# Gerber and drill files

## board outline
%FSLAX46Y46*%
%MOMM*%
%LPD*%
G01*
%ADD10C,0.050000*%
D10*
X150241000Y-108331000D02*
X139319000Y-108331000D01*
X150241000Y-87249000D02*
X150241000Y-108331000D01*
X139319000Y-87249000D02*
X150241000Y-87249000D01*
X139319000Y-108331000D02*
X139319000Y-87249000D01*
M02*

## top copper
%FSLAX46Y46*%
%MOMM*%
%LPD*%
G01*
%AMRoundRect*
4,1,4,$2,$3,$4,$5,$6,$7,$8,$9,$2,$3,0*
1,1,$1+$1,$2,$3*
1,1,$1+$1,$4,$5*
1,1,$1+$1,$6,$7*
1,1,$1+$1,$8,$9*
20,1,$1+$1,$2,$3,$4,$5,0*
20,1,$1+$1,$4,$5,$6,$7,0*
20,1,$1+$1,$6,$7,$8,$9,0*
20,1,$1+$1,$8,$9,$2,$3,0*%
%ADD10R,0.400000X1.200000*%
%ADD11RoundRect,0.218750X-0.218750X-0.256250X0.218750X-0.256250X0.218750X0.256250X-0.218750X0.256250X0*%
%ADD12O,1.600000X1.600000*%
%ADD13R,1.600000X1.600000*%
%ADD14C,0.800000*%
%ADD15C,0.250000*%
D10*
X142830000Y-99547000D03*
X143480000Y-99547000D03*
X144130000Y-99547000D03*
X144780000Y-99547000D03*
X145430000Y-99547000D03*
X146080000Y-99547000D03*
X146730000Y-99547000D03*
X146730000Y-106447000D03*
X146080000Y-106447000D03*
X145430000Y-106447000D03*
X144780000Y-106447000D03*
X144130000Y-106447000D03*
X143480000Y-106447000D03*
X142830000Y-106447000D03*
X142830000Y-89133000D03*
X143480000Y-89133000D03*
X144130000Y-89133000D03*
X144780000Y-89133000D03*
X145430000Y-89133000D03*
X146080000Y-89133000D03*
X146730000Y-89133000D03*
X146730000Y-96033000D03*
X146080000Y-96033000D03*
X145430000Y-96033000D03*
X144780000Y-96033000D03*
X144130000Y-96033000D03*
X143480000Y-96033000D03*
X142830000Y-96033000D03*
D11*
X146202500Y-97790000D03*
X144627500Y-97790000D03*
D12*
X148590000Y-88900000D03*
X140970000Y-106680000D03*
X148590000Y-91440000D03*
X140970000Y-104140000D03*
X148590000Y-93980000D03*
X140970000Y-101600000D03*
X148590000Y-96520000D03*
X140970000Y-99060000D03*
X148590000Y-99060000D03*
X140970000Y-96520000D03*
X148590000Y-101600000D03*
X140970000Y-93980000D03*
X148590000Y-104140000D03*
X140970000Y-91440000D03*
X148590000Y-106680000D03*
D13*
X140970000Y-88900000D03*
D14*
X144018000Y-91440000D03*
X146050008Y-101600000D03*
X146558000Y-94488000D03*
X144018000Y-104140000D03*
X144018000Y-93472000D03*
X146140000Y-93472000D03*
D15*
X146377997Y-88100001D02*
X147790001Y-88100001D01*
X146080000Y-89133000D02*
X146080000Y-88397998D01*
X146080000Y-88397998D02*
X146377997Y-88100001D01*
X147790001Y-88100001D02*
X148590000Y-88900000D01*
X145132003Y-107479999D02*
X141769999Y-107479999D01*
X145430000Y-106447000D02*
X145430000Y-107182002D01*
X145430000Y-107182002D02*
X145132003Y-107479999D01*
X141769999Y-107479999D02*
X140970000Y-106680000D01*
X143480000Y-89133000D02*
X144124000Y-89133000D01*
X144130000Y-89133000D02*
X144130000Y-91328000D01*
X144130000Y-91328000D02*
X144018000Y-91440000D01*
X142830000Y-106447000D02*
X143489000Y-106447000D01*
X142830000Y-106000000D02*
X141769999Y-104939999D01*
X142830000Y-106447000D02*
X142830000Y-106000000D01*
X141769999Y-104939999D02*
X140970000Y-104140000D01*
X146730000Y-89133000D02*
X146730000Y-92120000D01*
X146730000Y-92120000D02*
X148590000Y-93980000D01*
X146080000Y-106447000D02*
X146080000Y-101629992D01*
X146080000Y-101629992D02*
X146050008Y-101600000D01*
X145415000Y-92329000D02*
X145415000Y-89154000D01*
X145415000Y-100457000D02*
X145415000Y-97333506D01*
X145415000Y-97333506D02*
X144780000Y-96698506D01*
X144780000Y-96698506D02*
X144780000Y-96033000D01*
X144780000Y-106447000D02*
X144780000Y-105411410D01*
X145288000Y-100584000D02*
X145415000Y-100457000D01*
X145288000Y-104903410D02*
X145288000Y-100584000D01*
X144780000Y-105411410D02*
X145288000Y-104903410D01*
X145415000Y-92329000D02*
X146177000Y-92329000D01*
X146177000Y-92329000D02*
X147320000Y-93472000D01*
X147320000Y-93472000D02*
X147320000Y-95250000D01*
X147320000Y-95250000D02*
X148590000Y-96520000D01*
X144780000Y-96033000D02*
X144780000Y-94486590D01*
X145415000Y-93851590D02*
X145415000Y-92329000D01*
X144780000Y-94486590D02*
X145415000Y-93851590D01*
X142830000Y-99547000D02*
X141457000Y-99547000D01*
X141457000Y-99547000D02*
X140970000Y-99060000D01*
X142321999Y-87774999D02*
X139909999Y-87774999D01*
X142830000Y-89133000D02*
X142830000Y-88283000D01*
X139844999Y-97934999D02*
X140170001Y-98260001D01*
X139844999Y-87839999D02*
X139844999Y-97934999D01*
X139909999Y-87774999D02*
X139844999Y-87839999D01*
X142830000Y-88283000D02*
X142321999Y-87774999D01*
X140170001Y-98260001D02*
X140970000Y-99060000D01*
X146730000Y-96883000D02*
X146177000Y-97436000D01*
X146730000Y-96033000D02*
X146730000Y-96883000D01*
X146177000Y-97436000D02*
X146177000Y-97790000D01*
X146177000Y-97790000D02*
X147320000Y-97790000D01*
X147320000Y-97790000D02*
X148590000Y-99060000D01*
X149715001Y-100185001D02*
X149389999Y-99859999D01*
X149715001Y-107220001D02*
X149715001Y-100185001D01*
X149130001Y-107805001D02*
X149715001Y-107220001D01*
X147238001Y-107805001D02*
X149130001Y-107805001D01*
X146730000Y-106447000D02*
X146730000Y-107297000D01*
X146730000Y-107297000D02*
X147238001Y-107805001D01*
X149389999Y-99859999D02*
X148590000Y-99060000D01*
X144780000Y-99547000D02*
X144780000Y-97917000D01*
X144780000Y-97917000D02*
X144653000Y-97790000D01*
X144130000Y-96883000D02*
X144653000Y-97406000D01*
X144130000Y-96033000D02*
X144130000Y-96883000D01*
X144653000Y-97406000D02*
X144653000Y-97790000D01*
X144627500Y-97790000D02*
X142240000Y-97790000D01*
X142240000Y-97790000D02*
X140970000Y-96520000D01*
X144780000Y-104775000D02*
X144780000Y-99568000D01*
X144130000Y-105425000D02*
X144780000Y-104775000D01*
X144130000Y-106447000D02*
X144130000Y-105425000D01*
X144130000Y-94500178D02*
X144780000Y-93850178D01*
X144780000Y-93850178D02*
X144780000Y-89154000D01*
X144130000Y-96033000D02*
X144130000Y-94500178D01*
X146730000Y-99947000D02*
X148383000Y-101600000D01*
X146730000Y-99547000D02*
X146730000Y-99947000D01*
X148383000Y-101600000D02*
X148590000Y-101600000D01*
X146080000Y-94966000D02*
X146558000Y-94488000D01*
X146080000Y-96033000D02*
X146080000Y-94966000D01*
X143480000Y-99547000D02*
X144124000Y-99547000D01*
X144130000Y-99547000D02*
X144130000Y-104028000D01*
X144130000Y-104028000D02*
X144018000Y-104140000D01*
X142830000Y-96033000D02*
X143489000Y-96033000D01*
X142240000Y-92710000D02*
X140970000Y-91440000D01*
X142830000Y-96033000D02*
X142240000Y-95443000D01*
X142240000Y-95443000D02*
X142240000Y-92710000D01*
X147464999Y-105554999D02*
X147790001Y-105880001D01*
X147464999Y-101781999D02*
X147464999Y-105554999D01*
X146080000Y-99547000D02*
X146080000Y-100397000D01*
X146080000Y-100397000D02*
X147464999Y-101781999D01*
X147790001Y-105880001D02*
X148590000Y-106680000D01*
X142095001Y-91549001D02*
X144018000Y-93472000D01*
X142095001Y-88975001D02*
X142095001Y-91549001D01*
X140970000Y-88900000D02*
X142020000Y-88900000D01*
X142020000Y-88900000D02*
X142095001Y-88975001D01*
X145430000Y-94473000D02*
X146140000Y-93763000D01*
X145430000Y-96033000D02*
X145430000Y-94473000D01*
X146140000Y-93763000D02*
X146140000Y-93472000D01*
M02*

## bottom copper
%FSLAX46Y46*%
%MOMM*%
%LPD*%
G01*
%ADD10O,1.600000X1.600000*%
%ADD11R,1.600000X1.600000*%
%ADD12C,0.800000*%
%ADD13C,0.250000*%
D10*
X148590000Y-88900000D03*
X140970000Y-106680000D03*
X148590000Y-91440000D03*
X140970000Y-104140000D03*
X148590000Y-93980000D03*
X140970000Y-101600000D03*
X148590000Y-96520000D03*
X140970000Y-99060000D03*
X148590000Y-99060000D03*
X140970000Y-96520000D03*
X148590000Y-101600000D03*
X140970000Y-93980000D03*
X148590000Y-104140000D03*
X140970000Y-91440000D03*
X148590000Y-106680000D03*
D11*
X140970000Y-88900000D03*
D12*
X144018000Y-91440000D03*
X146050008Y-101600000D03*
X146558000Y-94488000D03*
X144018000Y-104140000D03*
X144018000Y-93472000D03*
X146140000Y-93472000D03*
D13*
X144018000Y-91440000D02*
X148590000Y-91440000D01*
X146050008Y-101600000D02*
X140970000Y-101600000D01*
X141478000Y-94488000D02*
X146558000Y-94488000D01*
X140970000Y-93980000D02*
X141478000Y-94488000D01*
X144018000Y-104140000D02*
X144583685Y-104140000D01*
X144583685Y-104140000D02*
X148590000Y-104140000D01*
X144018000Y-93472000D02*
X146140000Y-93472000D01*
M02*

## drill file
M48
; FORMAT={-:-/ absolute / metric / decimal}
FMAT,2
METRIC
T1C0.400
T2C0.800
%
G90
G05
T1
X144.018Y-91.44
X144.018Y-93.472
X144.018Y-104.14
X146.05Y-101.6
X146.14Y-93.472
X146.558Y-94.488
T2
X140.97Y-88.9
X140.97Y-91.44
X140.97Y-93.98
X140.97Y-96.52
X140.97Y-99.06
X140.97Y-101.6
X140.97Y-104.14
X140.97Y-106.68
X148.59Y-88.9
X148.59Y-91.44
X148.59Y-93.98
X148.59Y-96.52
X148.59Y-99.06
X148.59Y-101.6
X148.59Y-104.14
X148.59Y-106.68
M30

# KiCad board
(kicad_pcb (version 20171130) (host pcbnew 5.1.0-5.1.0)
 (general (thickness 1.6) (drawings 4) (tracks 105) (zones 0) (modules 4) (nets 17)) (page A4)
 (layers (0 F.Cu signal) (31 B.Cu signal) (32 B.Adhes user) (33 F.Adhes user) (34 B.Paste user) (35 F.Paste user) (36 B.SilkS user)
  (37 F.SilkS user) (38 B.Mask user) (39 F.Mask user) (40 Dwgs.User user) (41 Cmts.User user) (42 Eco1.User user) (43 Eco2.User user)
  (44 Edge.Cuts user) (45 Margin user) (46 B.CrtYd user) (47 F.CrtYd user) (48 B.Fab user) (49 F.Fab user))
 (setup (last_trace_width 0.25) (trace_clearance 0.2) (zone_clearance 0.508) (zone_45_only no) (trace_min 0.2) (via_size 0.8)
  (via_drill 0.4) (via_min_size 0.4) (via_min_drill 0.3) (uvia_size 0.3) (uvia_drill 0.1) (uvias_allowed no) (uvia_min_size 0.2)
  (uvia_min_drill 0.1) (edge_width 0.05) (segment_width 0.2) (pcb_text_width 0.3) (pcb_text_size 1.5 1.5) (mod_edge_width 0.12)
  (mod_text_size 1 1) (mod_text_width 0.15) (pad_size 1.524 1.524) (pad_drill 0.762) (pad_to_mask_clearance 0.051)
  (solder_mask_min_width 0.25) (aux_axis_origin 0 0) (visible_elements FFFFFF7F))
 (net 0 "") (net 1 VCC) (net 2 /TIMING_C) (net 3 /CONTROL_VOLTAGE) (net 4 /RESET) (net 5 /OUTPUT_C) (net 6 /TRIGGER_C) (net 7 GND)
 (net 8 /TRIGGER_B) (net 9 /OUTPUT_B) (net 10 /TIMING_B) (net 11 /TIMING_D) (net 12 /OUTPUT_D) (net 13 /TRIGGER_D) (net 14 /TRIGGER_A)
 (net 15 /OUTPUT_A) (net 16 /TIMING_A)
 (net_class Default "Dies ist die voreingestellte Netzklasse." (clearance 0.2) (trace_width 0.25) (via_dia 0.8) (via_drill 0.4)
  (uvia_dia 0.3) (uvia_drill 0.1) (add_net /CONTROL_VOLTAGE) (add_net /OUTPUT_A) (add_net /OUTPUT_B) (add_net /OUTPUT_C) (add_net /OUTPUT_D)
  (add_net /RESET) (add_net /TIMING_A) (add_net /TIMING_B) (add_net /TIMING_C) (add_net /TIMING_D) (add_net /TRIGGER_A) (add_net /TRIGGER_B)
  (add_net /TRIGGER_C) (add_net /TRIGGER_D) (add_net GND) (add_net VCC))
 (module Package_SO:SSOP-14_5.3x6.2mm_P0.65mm (layer F.Cu) (at 144.78 102.997 90)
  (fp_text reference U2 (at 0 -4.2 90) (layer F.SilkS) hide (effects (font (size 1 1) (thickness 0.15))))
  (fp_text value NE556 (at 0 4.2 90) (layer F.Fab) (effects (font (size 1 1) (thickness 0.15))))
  (pad 14 smd rect (at 3.45 -1.95 90) (size 1.2 0.4) (layers F.Cu F.Paste F.Mask) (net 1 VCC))
  (pad 13 smd rect (at 3.45 -1.3 90) (size 1.2 0.4) (layers F.Cu F.Paste F.Mask) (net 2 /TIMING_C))
  (pad 12 smd rect (at 3.45 -0.65 90) (size 1.2 0.4) (layers F.Cu F.Paste F.Mask) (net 2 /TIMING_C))
  (pad 11 smd rect (at 3.45 0 90) (size 1.2 0.4) (layers F.Cu F.Paste F.Mask) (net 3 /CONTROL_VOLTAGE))
  (pad 10 smd rect (at 3.45 0.65 90) (size 1.2 0.4) (layers F.Cu F.Paste F.Mask) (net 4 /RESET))
  (pad 9 smd rect (at 3.45 1.3 90) (size 1.2 0.4) (layers F.Cu F.Paste F.Mask) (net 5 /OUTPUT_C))
  (pad 8 smd rect (at 3.45 1.95 90) (size 1.2 0.4) (layers F.Cu F.Paste F.Mask) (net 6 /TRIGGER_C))
  (pad 7 smd rect (at -3.45 1.95 90) (size 1.2 0.4) (layers F.Cu F.Paste F.Mask) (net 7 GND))
  (pad 6 smd rect (at -3.45 1.3 90) (size 1.2 0.4) (layers F.Cu F.Paste F.Mask) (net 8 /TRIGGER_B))
  (pad 5 smd rect (at -3.45 0.65 90) (size 1.2 0.4) (layers F.Cu F.Paste F.Mask) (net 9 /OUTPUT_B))
  (pad 4 smd rect (at -3.45 0 90) (size 1.2 0.4) (layers F.Cu F.Paste F.Mask) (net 4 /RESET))
  (pad 3 smd rect (at -3.45 -0.65 90) (size 1.2 0.4) (layers F.Cu F.Paste F.Mask) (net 3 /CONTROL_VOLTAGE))
  (pad 2 smd rect (at -3.45 -1.3 90) (size 1.2 0.4) (layers F.Cu F.Paste F.Mask) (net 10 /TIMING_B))
  (pad 1 smd rect (at -3.45 -1.95 90) (size 1.2 0.4) (layers F.Cu F.Paste F.Mask) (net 10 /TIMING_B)))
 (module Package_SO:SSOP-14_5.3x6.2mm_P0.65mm (layer F.Cu) (at 144.78 92.583 90)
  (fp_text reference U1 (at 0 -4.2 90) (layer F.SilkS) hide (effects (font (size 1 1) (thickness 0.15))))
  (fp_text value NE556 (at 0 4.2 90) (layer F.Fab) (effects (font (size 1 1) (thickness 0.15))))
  (pad 14 smd rect (at 3.45 -1.95 90) (size 1.2 0.4) (layers F.Cu F.Paste F.Mask) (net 1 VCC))
  (pad 13 smd rect (at 3.45 -1.3 90) (size 1.2 0.4) (layers F.Cu F.Paste F.Mask) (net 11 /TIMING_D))
  (pad 12 smd rect (at 3.45 -0.65 90) (size 1.2 0.4) (layers F.Cu F.Paste F.Mask) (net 11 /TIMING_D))
  (pad 11 smd rect (at 3.45 0 90) (size 1.2 0.4) (layers F.Cu F.Paste F.Mask) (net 3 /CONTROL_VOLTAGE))
  (pad 10 smd rect (at 3.45 0.65 90) (size 1.2 0.4) (layers F.Cu F.Paste F.Mask) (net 4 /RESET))
  (pad 9 smd rect (at 3.45 1.3 90) (size 1.2 0.4) (layers F.Cu F.Paste F.Mask) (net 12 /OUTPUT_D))
  (pad 8 smd rect (at 3.45 1.95 90) (size 1.2 0.4) (layers F.Cu F.Paste F.Mask) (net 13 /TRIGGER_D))
  (pad 7 smd rect (at -3.45 1.95 90) (size 1.2 0.4) (layers F.Cu F.Paste F.Mask) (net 7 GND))
  (pad 6 smd rect (at -3.45 1.3 90) (size 1.2 0.4) (layers F.Cu F.Paste F.Mask) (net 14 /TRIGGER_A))
  (pad 5 smd rect (at -3.45 0.65 90) (size 1.2 0.4) (layers F.Cu F.Paste F.Mask) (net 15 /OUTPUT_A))
  (pad 4 smd rect (at -3.45 0 90) (size 1.2 0.4) (layers F.Cu F.Paste F.Mask) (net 4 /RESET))
  (pad 3 smd rect (at -3.45 -0.65 90) (size 1.2 0.4) (layers F.Cu F.Paste F.Mask) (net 3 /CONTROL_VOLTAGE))
  (pad 2 smd rect (at -3.45 -1.3 90) (size 1.2 0.4) (layers F.Cu F.Paste F.Mask) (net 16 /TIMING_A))
  (pad 1 smd rect (at -3.45 -1.95 90) (size 1.2 0.4) (layers F.Cu F.Paste F.Mask) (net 16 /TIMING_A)))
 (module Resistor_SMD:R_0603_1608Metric (layer F.Cu) (at 145.415 97.79)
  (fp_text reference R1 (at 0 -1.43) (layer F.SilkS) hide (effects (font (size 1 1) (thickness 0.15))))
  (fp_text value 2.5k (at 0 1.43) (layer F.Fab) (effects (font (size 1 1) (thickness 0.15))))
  (pad 2 smd roundrect (at 0.7875 0) (size 0.875 0.95) (layers F.Cu F.Paste F.Mask) (roundrect_rratio 0.25) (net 7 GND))
  (pad 1 smd roundrect (at -0.7875 0) (size 0.875 0.95) (layers F.Cu F.Paste F.Mask) (roundrect_rratio 0.25) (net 3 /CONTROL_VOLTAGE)))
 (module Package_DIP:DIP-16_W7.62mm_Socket (layer F.Cu) (at 140.97 88.9)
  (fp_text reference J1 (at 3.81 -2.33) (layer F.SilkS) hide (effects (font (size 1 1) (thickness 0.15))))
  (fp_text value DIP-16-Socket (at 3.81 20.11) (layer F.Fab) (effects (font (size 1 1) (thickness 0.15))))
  (pad 16 thru_hole oval (at 7.62 0) (size 1.6 1.6) (drill 0.8) (layers *.Cu *.Mask) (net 12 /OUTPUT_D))
  (pad 8 thru_hole oval (at 0 17.78) (size 1.6 1.6) (drill 0.8) (layers *.Cu *.Mask) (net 9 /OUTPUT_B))
  (pad 15 thru_hole oval (at 7.62 2.54) (size 1.6 1.6) (drill 0.8) (layers *.Cu *.Mask) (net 11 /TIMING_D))
  (pad 7 thru_hole oval (at 0 15.24) (size 1.6 1.6) (drill 0.8) (layers *.Cu *.Mask) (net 10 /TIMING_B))
  (pad 14 thru_hole oval (at 7.62 5.08) (size 1.6 1.6) (drill 0.8) (layers *.Cu *.Mask) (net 13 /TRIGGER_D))
  (pad 6 thru_hole oval (at 0 12.7) (size 1.6 1.6) (drill 0.8) (layers *.Cu *.Mask) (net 8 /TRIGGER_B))
  (pad 13 thru_hole oval (at 7.62 7.62) (size 1.6 1.6) (drill 0.8) (layers *.Cu *.Mask) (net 4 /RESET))
  (pad 5 thru_hole oval (at 0 10.16) (size 1.6 1.6) (drill 0.8) (layers *.Cu *.Mask) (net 1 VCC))
  (pad 12 thru_hole oval (at 7.62 10.16) (size 1.6 1.6) (drill 0.8) (layers *.Cu *.Mask) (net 7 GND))
  (pad 4 thru_hole oval (at 0 7.62) (size 1.6 1.6) (drill 0.8) (layers *.Cu *.Mask) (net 3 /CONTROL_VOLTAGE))
  (pad 11 thru_hole oval (at 7.62 12.7) (size 1.6 1.6) (drill 0.8) (layers *.Cu *.Mask) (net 6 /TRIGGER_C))
  (pad 3 thru_hole oval (at 0 5.08) (size 1.6 1.6) (drill 0.8) (layers *.Cu *.Mask) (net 14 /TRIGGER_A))
  (pad 10 thru_hole oval (at 7.62 15.24) (size 1.6 1.6) (drill 0.8) (layers *.Cu *.Mask) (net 2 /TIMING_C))
  (pad 2 thru_hole oval (at 0 2.54) (size 1.6 1.6) (drill 0.8) (layers *.Cu *.Mask) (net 16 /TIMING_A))
  (pad 9 thru_hole oval (at 7.62 17.78) (size 1.6 1.6) (drill 0.8) (layers *.Cu *.Mask) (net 5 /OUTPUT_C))
  (pad 1 thru_hole rect (at 0 0) (size 1.6 1.6) (drill 0.8) (layers *.Cu *.Mask) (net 15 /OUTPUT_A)))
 (gr_line (start 150.241 108.331) (end 139.319 108.331) (layer Edge.Cuts) (width 0.05))
 (gr_line (start 150.241 87.249) (end 150.241 108.331) (layer Edge.Cuts) (width 0.05))
 (gr_line (start 139.319 87.249) (end 150.241 87.249) (layer Edge.Cuts) (width 0.05))
 (gr_line (start 139.319 108.331) (end 139.319 87.249) (layer Edge.Cuts) (width 0.05))
 (segment (start 146.377997 88.100001) (end 147.790001 88.100001) (width 0.25) (layer F.Cu) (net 12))
 (segment (start 146.08 89.133) (end 146.08 88.397998) (width 0.25) (layer F.Cu) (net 12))
 (segment (start 146.08 88.397998) (end 146.377997 88.100001) (width 0.25) (layer F.Cu) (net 12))
 (segment (start 147.790001 88.100001) (end 148.59 88.9) (width 0.25) (layer F.Cu) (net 12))
 (segment (start 145.132003 107.479999) (end 141.769999 107.479999) (width 0.25) (layer F.Cu) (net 9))
 (segment (start 145.43 106.447) (end 145.43 107.182002) (width 0.25) (layer F.Cu) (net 9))
 (segment (start 145.43 107.182002) (end 145.132003 107.479999) (width 0.25) (layer F.Cu) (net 9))
 (segment (start 141.769999 107.479999) (end 140.97 106.68) (width 0.25) (layer F.Cu) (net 9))
 (segment (start 143.48 89.133) (end 144.124 89.133) (width 0.25) (layer F.Cu) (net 11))
 (via (at 144.018 91.44) (size 0.8) (drill 0.4) (layers F.Cu B.Cu) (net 11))
 (segment (start 144.13 89.133) (end 144.13 91.328) (width 0.25) (layer F.Cu) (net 11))
 (segment (start 144.13 91.328) (end 144.018 91.44) (width 0.25) (layer F.Cu) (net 11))
 (segment (start 144.018 91.44) (end 148.59 91.44) (width 0.25) (layer B.Cu) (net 11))
 (segment (start 142.83 106.447) (end 143.489 106.447) (width 0.25) (layer F.Cu) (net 10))
 (segment (start 142.83 106) (end 141.769999 104.939999) (width 0.25) (layer F.Cu) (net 10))
 (segment (start 142.83 106.447) (end 142.83 106) (width 0.25) (layer F.Cu) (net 10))
 (segment (start 141.769999 104.939999) (end 140.97 104.14) (width 0.25) (layer F.Cu) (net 10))
 (segment (start 146.73 89.133) (end 146.73 92.12) (width 0.25) (layer F.Cu) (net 13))
 (segment (start 146.73 92.12) (end 148.59 93.98) (width 0.25) (layer F.Cu) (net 13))
 (via (at 146.050008 101.6) (size 0.8) (drill 0.4) (layers F.Cu B.Cu) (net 8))
 (segment (start 146.08 106.447) (end 146.08 101.629992) (width 0.25) (layer F.Cu) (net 8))
 (segment (start 146.08 101.629992) (end 146.050008 101.6) (width 0.25) (layer F.Cu) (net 8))
 (segment (start 146.050008 101.6) (end 140.97 101.6) (width 0.25) (layer B.Cu) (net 8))
 (segment (start 145.415 92.329) (end 145.415 89.154) (width 0.25) (layer F.Cu) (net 4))
 (segment (start 145.415 100.457) (end 145.415 97.333506) (width 0.25) (layer F.Cu) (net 4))
 (segment (start 145.415 97.333506) (end 144.78 96.698506) (width 0.25) (layer F.Cu) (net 4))
 (segment (start 144.78 96.698506) (end 144.78 96.033) (width 0.25) (layer F.Cu) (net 4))
 (segment (start 144.78 106.447) (end 144.78 105.41141) (width 0.25) (layer F.Cu) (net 4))
 (segment (start 145.288 100.584) (end 145.415 100.457) (width 0.25) (layer F.Cu) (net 4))
 (segment (start 145.288 104.90341) (end 145.288 100.584) (width 0.25) (layer F.Cu) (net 4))
 (segment (start 144.78 105.41141) (end 145.288 104.90341) (width 0.25) (layer F.Cu) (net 4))
 (segment (start 145.415 92.329) (end 146.177 92.329) (width 0.25) (layer F.Cu) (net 4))
 (segment (start 146.177 92.329) (end 147.32 93.472) (width 0.25) (layer F.Cu) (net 4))
 (segment (start 147.32 93.472) (end 147.32 95.25) (width 0.25) (layer F.Cu) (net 4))
 (segment (start 147.32 95.25) (end 148.59 96.52) (width 0.25) (layer F.Cu) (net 4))
 (segment (start 144.78 96.033) (end 144.78 94.48659) (width 0.25) (layer F.Cu) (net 4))
 (segment (start 145.415 93.85159) (end 145.415 92.329) (width 0.25) (layer F.Cu) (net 4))
 (segment (start 144.78 94.48659) (end 145.415 93.85159) (width 0.25) (layer F.Cu) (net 4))
 (segment (start 142.83 99.547) (end 141.457 99.547) (width 0.25) (layer F.Cu) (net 1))
 (segment (start 141.457 99.547) (end 140.97 99.06) (width 0.25) (layer F.Cu) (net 1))
 (segment (start 142.321999 87.774999) (end 139.909999 87.774999) (width 0.25) (layer F.Cu) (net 1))
 (segment (start 142.83 89.133) (end 142.83 88.283) (width 0.25) (layer F.Cu) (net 1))
 (segment (start 139.844999 97.934999) (end 140.170001 98.260001) (width 0.25) (layer F.Cu) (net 1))
 (segment (start 139.844999 87.839999) (end 139.844999 97.934999) (width 0.25) (layer F.Cu) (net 1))
 (segment (start 139.909999 87.774999) (end 139.844999 87.839999) (width 0.25) (layer F.Cu) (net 1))
 (segment (start 142.83 88.283) (end 142.321999 87.774999) (width 0.25) (layer F.Cu) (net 1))
 (segment (start 140.170001 98.260001) (end 140.97 99.06) (width 0.25) (layer F.Cu) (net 1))
 (segment (start 146.73 96.883) (end 146.177 97.436) (width 0.25) (layer F.Cu) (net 7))
 (segment (start 146.73 96.033) (end 146.73 96.883) (width 0.25) (layer F.Cu) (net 7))
 (segment (start 146.177 97.436) (end 146.177 97.79) (width 0.25) (layer F.Cu) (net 7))
 (segment (start 146.177 97.79) (end 147.32 97.79) (width 0.25) (layer F.Cu) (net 7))
 (segment (start 147.32 97.79) (end 148.59 99.06) (width 0.25) (layer F.Cu) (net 7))
 (segment (start 149.715001 100.185001) (end 149.389999 99.859999) (width 0.25) (layer F.Cu) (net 7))
 (segment (start 149.715001 107.220001) (end 149.715001 100.185001) (width 0.25) (layer F.Cu) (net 7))
 (segment (start 149.130001 107.805001) (end 149.715001 107.220001) (width 0.25) (layer F.Cu) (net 7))
 (segment (start 147.238001 107.805001) (end 149.130001 107.805001) (width 0.25) (layer F.Cu) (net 7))
 (segment (start 146.73 106.447) (end 146.73 107.297) (width 0.25) (layer F.Cu) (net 7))
 (segment (start 146.73 107.297) (end 147.238001 107.805001) (width 0.25) (layer F.Cu) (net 7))
 (segment (start 149.389999 99.859999) (end 148.59 99.06) (width 0.25) (layer F.Cu) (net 7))
 (segment (start 144.78 99.547) (end 144.78 97.917) (width 0.25) (layer F.Cu) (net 3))
 (segment (start 144.78 97.917) (end 144.653 97.79) (width 0.25) (layer F.Cu) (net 3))
 (segment (start 144.13 96.883) (end 144.653 97.406) (width 0.25) (layer F.Cu) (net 3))
 (segment (start 144.13 96.033) (end 144.13 96.883) (width 0.25) (layer F.Cu) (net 3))
 (segment (start 144.653 97.406) (end 144.653 97.79) (width 0.25) (layer F.Cu) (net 3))
 (segment (start 144.6275 97.79) (end 142.24 97.79) (width 0.25) (layer F.Cu) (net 3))
 (segment (start 142.24 97.79) (end 140.97 96.52) (width 0.25) (layer F.Cu) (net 3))
 (segment (start 144.78 104.775) (end 144.78 99.568) (width 0.25) (layer F.Cu) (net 3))
 (segment (start 144.13 105.425) (end 144.78 104.775) (width 0.25) (layer F.Cu) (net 3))
 (segment (start 144.13 106.447) (end 144.13 105.425) (width 0.25) (layer F.Cu) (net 3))
 (segment (start 144.13 94.500178) (end 144.78 93.850178) (width 0.25) (layer F.Cu) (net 3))
 (segment (start 144.78 93.850178) (end 144.78 89.154) (width 0.25) (layer F.Cu) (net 3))
 (segment (start 144.13 96.033) (end 144.13 94.500178) (width 0.25) (layer F.Cu) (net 3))
 (segment (start 146.73 99.947) (end 148.383 101.6) (width 0.25) (layer F.Cu) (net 6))
 (segment (start 146.73 99.547) (end 146.73 99.947) (width 0.25) (layer F.Cu) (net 6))
 (segment (start 148.383 101.6) (end 148.59 101.6) (width 0.25) (layer F.Cu) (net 6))
 (via (at 146.558 94.488) (size 0.8) (drill 0.4) (layers F.Cu B.Cu) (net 14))
 (segment (start 146.08 94.966) (end 146.558 94.488) (width 0.25) (layer F.Cu) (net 14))
 (segment (start 146.08 96.033) (end 146.08 94.966) (width 0.25) (layer F.Cu) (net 14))
 (segment (start 141.478 94.488) (end 146.558 94.488) (width 0.25) (layer B.Cu) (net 14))
 (segment (start 140.97 93.98) (end 141.478 94.488) (width 0.25) (layer B.Cu) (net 14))
 (segment (start 143.48 99.547) (end 144.124 99.547) (width 0.25) (layer F.Cu) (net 2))
 (segment (start 144.13 99.547) (end 144.13 104.028) (width 0.25) (layer F.Cu) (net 2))
 (via (at 144.018 104.14) (size 0.8) (drill 0.4) (layers F.Cu B.Cu) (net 2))
 (segment (start 144.13 104.028) (end 144.018 104.14) (width 0.25) (layer F.Cu) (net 2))
 (segment (start 144.018 104.14) (end 144.583685 104.14) (width 0.25) (layer B.Cu) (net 2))
 (segment (start 144.583685 104.14) (end 148.59 104.14) (width 0.25) (layer B.Cu) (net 2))
 (segment (start 142.83 96.033) (end 143.489 96.033) (width 0.25) (layer F.Cu) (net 16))
 (segment (start 142.24 92.71) (end 140.97 91.44) (width 0.25) (layer F.Cu) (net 16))
 (segment (start 142.83 96.033) (end 142.24 95.443) (width 0.25) (layer F.Cu) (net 16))
 (segment (start 142.24 95.443) (end 142.24 92.71) (width 0.25) (layer F.Cu) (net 16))
 (segment (start 147.464999 105.554999) (end 147.790001 105.880001) (width 0.25) (layer F.Cu) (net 5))
 (segment (start 147.464999 101.781999) (end 147.464999 105.554999) (width 0.25) (layer F.Cu) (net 5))
 (segment (start 146.08 99.547) (end 146.08 100.397) (width 0.25) (layer F.Cu) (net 5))
 (segment (start 146.08 100.397) (end 147.464999 101.781999) (width 0.25) (layer F.Cu) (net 5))
 (segment (start 147.790001 105.880001) (end 148.59 106.68) (width 0.25) (layer F.Cu) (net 5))
 (segment (start 142.095001 91.549001) (end 144.018 93.472) (width 0.25) (layer F.Cu) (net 15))
 (segment (start 142.095001 88.975001) (end 142.095001 91.549001) (width 0.25) (layer F.Cu) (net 15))
 (via (at 144.018 93.472) (size 0.8) (drill 0.4) (layers F.Cu B.Cu) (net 15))
 (segment (start 140.97 88.9) (end 142.02 88.9) (width 0.25) (layer F.Cu) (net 15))
 (segment (start 142.02 88.9) (end 142.095001 88.975001) (width 0.25) (layer F.Cu) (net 15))
 (via (at 146.14 93.472) (size 0.8) (drill 0.4) (layers F.Cu B.Cu) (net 15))
 (segment (start 144.018 93.472) (end 146.14 93.472) (width 0.25) (layer B.Cu) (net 15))
 (segment (start 145.43 94.473) (end 146.14 93.763) (width 0.25) (layer F.Cu) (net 15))
 (segment (start 145.43 96.033) (end 145.43 94.473) (width 0.25) (layer F.Cu) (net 15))
 (segment (start 146.14 93.763) (end 146.14 93.472) (width 0.25) (layer F.Cu) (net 15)))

